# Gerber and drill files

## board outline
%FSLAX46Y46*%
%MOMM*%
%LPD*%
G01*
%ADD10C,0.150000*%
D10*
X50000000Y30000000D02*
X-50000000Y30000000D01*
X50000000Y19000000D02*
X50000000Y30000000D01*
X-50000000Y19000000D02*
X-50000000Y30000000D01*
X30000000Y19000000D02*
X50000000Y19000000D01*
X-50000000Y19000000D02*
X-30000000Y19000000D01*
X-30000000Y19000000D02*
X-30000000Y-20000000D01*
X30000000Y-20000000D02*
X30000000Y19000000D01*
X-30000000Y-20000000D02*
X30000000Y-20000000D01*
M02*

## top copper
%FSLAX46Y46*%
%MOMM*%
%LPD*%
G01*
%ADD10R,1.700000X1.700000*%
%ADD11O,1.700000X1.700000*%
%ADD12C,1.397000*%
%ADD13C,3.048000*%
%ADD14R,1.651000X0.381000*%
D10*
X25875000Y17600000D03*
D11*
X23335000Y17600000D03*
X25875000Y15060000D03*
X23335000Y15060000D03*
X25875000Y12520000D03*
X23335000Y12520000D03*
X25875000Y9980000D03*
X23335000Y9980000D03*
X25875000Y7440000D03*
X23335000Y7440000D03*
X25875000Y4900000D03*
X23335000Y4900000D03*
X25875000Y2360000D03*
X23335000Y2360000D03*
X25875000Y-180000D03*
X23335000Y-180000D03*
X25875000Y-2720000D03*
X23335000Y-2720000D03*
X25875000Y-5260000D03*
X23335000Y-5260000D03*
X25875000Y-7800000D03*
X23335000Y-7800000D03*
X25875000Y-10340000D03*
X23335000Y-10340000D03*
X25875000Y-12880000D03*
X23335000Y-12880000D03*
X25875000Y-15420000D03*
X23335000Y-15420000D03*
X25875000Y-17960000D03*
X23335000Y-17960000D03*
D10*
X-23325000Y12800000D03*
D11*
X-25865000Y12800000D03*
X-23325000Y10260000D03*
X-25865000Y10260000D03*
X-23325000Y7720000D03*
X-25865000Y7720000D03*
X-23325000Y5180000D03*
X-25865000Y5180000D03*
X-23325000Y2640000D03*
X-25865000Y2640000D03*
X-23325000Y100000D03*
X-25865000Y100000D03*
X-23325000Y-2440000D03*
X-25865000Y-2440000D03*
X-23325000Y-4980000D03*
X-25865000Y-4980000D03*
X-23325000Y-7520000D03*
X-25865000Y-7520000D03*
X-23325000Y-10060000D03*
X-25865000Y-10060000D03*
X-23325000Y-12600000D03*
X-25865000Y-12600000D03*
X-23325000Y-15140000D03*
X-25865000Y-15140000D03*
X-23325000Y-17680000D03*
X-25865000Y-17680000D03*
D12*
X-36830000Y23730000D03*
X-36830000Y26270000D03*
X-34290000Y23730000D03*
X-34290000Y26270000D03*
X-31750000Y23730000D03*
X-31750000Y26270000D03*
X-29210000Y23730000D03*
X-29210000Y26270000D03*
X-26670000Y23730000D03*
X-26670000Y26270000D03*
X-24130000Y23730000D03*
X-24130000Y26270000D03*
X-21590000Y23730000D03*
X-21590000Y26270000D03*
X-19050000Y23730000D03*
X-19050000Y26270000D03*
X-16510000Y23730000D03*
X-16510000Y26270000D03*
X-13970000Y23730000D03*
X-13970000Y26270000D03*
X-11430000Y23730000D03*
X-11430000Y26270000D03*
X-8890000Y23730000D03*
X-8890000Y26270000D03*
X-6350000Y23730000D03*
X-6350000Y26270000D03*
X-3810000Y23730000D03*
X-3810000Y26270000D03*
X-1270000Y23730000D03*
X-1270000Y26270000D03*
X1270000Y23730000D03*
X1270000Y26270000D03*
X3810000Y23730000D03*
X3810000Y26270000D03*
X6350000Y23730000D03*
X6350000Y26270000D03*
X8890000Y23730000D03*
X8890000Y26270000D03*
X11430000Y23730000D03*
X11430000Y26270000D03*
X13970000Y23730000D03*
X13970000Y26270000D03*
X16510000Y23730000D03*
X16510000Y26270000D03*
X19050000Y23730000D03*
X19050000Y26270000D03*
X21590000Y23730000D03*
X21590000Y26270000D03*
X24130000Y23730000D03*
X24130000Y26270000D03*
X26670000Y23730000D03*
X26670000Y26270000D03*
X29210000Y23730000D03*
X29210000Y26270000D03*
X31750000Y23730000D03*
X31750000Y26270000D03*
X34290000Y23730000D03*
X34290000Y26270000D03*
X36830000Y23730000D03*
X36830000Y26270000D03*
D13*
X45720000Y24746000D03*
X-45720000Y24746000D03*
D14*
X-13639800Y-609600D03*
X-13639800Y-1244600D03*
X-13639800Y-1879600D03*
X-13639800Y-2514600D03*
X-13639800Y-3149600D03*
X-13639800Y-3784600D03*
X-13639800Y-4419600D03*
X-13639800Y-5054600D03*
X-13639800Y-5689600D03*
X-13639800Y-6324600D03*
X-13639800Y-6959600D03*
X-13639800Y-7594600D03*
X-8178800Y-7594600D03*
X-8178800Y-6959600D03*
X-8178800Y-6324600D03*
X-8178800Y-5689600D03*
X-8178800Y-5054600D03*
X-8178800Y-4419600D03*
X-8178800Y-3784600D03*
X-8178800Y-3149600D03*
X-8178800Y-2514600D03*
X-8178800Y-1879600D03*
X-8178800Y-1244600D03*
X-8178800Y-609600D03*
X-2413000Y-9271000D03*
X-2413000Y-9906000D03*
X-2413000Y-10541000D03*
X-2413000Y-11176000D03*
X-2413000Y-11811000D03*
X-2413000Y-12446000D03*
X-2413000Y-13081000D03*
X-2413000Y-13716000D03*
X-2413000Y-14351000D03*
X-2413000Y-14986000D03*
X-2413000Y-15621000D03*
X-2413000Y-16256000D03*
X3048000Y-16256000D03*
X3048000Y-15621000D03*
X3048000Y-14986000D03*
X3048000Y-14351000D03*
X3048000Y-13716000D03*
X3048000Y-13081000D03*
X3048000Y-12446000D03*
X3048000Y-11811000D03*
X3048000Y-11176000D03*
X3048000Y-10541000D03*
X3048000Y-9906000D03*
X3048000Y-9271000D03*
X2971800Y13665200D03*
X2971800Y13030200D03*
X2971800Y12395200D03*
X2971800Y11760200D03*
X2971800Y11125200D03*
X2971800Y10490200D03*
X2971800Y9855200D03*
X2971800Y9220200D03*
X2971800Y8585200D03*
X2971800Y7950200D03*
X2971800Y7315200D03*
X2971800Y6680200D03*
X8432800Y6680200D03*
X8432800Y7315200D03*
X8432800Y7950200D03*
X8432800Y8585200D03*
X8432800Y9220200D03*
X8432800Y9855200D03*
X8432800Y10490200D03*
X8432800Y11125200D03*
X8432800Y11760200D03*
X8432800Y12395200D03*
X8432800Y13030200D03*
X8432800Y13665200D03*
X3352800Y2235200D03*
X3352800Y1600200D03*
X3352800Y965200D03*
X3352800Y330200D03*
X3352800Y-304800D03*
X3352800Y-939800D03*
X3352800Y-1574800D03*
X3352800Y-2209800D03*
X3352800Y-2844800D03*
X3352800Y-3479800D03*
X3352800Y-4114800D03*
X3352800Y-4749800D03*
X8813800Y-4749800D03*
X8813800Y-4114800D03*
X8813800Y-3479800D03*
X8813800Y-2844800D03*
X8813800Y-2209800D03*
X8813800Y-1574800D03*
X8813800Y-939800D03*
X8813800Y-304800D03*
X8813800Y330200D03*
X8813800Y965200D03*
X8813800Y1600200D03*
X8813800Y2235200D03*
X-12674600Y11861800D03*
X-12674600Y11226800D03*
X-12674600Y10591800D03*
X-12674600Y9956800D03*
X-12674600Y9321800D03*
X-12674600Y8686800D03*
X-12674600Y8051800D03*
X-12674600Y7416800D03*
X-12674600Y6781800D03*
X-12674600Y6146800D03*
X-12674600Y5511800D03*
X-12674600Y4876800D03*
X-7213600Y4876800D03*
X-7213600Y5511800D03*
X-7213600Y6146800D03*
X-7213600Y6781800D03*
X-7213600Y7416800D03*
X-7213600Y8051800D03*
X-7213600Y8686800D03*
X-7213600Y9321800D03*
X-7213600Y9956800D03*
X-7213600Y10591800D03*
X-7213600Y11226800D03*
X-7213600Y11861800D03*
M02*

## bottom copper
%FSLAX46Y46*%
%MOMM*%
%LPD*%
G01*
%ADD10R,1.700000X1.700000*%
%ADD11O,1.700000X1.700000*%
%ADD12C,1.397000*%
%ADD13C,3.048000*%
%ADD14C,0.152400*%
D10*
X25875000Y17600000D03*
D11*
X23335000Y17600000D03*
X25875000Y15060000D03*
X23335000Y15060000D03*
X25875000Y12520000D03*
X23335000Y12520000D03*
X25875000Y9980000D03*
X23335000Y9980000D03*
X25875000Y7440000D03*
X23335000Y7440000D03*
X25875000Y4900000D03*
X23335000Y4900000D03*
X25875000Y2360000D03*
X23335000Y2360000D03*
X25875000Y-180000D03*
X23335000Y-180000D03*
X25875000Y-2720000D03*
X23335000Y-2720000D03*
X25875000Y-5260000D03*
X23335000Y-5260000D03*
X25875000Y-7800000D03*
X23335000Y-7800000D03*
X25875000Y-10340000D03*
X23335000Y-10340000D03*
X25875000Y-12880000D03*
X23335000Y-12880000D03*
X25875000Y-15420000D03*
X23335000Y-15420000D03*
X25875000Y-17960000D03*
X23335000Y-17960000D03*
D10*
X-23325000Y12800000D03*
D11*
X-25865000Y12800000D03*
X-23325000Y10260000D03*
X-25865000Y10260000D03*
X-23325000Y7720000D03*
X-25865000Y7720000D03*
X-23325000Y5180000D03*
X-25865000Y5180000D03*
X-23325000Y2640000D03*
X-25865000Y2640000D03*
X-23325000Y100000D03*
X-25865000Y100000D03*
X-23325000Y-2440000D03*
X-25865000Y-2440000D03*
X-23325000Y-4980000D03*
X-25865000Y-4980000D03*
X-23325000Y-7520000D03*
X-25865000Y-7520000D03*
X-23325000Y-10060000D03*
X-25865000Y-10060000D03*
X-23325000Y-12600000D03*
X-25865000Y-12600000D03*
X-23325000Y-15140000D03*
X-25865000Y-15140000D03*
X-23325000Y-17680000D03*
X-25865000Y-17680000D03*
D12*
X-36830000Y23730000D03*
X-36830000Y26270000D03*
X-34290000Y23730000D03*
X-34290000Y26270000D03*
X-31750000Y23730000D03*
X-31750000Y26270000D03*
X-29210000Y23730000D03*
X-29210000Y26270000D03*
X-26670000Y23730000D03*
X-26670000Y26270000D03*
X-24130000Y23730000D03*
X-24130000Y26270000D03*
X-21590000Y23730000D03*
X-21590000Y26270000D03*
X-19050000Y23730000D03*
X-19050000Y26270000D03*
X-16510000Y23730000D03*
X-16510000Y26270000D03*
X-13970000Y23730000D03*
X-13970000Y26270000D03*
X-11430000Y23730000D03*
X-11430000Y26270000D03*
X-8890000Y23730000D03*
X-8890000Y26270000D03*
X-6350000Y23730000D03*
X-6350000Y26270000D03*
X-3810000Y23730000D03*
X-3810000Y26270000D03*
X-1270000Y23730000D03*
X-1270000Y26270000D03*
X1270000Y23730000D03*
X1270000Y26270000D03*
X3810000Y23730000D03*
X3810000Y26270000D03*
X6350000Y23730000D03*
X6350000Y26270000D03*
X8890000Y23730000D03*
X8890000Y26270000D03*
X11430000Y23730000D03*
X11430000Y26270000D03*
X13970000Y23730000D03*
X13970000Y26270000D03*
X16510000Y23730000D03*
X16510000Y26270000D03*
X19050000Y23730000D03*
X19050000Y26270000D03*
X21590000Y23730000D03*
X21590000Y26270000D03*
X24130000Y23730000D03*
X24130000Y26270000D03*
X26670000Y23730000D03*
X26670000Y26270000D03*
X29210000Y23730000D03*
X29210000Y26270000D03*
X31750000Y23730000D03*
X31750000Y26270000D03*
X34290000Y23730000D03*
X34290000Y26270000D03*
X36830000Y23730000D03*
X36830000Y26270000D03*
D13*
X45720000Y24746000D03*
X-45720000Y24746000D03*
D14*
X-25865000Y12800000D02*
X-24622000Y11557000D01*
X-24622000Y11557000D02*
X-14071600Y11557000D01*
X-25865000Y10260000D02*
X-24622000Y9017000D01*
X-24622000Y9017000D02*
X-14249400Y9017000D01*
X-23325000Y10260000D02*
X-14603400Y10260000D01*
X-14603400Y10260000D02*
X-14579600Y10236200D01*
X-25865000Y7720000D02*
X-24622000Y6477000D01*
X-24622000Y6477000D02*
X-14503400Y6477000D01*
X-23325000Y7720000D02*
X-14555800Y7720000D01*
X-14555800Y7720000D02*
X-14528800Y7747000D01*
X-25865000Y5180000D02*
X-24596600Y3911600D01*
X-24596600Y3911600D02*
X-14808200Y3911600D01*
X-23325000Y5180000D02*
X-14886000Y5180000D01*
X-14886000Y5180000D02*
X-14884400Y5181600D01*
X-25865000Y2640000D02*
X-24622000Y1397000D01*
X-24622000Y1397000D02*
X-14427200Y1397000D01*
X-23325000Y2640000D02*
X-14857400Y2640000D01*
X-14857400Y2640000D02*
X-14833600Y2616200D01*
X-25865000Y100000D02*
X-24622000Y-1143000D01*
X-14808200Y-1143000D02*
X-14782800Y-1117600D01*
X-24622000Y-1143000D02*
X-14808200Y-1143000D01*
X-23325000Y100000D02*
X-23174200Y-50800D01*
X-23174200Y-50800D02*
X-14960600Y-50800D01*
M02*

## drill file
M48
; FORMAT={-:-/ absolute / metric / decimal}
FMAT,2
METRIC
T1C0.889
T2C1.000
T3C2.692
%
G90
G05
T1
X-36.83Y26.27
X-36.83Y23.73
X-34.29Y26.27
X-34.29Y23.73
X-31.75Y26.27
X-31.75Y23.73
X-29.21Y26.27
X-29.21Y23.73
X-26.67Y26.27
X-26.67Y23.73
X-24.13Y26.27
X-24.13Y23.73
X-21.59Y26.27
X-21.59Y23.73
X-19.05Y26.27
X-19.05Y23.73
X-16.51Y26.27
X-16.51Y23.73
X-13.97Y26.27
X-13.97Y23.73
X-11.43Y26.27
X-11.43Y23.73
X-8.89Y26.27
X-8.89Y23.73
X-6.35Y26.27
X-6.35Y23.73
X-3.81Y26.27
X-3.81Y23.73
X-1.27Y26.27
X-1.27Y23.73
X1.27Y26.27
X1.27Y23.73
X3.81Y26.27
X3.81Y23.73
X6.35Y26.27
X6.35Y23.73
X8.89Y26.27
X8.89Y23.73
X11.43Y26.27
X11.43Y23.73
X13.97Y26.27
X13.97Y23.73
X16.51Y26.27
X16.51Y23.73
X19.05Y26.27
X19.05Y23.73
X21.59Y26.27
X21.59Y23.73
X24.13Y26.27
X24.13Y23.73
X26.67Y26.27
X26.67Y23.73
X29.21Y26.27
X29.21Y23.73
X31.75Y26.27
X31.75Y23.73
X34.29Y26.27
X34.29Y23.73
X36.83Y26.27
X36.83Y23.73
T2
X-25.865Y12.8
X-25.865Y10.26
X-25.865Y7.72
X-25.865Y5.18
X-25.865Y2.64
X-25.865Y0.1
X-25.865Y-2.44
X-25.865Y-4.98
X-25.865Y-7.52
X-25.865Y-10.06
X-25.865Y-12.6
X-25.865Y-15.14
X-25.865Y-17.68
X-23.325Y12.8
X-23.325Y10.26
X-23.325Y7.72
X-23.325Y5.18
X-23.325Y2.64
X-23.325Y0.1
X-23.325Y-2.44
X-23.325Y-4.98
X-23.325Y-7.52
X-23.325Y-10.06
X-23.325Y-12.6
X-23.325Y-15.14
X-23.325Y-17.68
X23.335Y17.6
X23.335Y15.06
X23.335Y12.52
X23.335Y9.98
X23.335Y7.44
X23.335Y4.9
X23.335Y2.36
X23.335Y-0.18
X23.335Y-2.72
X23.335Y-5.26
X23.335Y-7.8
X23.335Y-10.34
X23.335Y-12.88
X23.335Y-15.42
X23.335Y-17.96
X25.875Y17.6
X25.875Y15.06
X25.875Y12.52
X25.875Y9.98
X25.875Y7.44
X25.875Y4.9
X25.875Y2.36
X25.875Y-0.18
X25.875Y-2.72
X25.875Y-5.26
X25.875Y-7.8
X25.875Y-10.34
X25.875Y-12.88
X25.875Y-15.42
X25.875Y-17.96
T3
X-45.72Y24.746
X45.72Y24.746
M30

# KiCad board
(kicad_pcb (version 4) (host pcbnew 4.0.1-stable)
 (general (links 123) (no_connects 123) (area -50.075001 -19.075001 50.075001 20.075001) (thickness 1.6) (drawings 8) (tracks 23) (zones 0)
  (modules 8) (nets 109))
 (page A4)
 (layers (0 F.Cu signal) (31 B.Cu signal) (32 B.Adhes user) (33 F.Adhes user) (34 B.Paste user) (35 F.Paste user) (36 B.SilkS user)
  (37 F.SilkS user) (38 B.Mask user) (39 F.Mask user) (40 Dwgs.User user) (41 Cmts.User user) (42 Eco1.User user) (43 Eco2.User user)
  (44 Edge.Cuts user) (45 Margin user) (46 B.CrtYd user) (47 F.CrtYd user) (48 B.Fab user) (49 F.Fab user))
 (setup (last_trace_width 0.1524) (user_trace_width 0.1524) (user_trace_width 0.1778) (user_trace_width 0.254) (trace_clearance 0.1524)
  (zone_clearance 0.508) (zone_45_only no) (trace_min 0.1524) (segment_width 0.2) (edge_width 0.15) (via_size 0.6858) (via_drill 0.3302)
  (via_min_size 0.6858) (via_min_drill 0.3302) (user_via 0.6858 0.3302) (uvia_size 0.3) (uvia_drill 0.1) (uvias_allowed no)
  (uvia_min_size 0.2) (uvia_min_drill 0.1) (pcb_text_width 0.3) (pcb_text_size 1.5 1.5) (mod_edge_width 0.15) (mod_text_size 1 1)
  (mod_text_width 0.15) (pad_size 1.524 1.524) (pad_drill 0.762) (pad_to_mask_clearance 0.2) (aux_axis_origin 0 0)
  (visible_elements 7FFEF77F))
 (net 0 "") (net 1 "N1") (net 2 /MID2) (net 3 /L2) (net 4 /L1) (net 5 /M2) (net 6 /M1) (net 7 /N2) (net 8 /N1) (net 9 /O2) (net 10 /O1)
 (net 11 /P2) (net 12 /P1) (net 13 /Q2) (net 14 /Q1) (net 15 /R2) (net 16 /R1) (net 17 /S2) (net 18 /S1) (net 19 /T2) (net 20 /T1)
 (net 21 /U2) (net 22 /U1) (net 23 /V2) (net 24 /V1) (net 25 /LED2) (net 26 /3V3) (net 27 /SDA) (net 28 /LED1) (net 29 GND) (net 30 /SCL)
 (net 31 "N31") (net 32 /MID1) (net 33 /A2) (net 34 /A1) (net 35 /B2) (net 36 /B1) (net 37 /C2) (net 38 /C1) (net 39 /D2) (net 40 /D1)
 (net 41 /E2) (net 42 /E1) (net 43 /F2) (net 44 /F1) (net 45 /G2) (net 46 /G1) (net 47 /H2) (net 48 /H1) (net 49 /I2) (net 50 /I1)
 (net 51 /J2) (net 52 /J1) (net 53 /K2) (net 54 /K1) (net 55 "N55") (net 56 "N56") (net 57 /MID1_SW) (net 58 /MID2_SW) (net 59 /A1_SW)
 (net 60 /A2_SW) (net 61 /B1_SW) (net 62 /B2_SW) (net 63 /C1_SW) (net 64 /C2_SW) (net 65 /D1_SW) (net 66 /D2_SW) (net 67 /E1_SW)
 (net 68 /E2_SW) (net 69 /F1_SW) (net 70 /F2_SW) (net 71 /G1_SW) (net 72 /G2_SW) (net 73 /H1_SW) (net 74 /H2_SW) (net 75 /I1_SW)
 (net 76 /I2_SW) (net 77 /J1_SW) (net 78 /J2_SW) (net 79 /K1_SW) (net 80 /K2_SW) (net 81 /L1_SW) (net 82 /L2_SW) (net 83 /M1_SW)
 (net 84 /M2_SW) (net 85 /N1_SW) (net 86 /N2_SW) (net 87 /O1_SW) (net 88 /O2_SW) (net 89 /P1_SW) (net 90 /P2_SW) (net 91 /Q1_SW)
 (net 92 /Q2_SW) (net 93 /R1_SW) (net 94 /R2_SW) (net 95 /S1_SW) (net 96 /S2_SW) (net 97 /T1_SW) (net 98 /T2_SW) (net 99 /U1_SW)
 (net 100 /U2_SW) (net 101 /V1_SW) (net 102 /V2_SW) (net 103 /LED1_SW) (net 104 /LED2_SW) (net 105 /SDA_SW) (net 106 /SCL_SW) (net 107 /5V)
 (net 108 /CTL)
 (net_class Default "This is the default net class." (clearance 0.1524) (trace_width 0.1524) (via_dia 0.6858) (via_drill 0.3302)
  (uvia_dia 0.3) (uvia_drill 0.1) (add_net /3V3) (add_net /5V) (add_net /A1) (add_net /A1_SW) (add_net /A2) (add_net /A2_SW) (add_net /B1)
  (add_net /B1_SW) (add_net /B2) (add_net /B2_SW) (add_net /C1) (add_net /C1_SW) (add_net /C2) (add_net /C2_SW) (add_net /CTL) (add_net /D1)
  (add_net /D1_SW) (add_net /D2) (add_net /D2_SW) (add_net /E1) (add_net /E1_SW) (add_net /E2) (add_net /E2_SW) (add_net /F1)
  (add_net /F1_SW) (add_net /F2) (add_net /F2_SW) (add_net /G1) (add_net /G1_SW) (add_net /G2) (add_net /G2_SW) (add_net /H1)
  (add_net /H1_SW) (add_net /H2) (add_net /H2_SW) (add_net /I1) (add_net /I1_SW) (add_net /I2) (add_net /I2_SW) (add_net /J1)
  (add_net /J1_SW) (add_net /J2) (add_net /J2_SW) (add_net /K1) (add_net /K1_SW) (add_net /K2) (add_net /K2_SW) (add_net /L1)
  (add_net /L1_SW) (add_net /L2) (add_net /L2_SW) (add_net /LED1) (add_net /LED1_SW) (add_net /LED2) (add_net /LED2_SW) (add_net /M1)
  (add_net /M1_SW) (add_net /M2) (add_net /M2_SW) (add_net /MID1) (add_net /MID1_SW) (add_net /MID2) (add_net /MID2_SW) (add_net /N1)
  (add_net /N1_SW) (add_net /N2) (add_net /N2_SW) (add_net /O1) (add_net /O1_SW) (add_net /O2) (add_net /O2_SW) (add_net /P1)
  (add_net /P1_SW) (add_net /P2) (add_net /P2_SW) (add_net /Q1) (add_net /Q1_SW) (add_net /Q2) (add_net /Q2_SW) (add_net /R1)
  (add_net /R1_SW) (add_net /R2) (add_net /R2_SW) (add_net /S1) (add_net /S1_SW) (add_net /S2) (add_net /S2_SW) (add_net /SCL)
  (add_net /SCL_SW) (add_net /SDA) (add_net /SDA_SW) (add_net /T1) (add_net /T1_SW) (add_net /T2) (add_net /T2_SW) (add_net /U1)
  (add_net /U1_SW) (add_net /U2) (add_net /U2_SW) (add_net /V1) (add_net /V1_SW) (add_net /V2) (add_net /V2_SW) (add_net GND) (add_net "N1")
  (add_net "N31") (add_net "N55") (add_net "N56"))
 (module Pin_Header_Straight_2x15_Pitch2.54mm (layer B.Cu) (at 24.605 0.18 180)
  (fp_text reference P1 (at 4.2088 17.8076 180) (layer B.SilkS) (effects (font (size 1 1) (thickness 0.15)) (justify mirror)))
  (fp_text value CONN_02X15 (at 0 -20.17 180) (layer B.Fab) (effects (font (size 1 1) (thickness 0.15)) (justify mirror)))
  (pad 1 thru_hole rect (at -1.27 17.78 180) (size 1.7 1.7) (drill 1) (layers *.Cu *.Mask) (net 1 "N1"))
  (pad 2 thru_hole oval (at 1.27 17.78 180) (size 1.7 1.7) (drill 1) (layers *.Cu *.Mask) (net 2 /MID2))
  (pad 3 thru_hole oval (at -1.27 15.24 180) (size 1.7 1.7) (drill 1) (layers *.Cu *.Mask) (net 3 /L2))
  (pad 4 thru_hole oval (at 1.27 15.24 180) (size 1.7 1.7) (drill 1) (layers *.Cu *.Mask) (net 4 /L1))
  (pad 5 thru_hole oval (at -1.27 12.7 180) (size 1.7 1.7) (drill 1) (layers *.Cu *.Mask) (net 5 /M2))
  (pad 6 thru_hole oval (at 1.27 12.7 180) (size 1.7 1.7) (drill 1) (layers *.Cu *.Mask) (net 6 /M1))
  (pad 7 thru_hole oval (at -1.27 10.16 180) (size 1.7 1.7) (drill 1) (layers *.Cu *.Mask) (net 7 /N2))
  (pad 8 thru_hole oval (at 1.27 10.16 180) (size 1.7 1.7) (drill 1) (layers *.Cu *.Mask) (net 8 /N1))
  (pad 9 thru_hole oval (at -1.27 7.62 180) (size 1.7 1.7) (drill 1) (layers *.Cu *.Mask) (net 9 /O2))
  (pad 10 thru_hole oval (at 1.27 7.62 180) (size 1.7 1.7) (drill 1) (layers *.Cu *.Mask) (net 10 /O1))
  (pad 11 thru_hole oval (at -1.27 5.08 180) (size 1.7 1.7) (drill 1) (layers *.Cu *.Mask) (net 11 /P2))
  (pad 12 thru_hole oval (at 1.27 5.08 180) (size 1.7 1.7) (drill 1) (layers *.Cu *.Mask) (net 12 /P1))
  (pad 13 thru_hole oval (at -1.27 2.54 180) (size 1.7 1.7) (drill 1) (layers *.Cu *.Mask) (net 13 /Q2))
  (pad 14 thru_hole oval (at 1.27 2.54 180) (size 1.7 1.7) (drill 1) (layers *.Cu *.Mask) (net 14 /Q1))
  (pad 15 thru_hole oval (at -1.27 0 180) (size 1.7 1.7) (drill 1) (layers *.Cu *.Mask) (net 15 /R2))
  (pad 16 thru_hole oval (at 1.27 0 180) (size 1.7 1.7) (drill 1) (layers *.Cu *.Mask) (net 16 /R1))
  (pad 17 thru_hole oval (at -1.27 -2.54 180) (size 1.7 1.7) (drill 1) (layers *.Cu *.Mask) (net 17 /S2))
  (pad 18 thru_hole oval (at 1.27 -2.54 180) (size 1.7 1.7) (drill 1) (layers *.Cu *.Mask) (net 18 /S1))
  (pad 19 thru_hole oval (at -1.27 -5.08 180) (size 1.7 1.7) (drill 1) (layers *.Cu *.Mask) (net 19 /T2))
  (pad 20 thru_hole oval (at 1.27 -5.08 180) (size 1.7 1.7) (drill 1) (layers *.Cu *.Mask) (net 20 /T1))
  (pad 21 thru_hole oval (at -1.27 -7.62 180) (size 1.7 1.7) (drill 1) (layers *.Cu *.Mask) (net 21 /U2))
  (pad 22 thru_hole oval (at 1.27 -7.62 180) (size 1.7 1.7) (drill 1) (layers *.Cu *.Mask) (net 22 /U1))
  (pad 23 thru_hole oval (at -1.27 -10.16 180) (size 1.7 1.7) (drill 1) (layers *.Cu *.Mask) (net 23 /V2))
  (pad 24 thru_hole oval (at 1.27 -10.16 180) (size 1.7 1.7) (drill 1) (layers *.Cu *.Mask) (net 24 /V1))
  (pad 25 thru_hole oval (at -1.27 -12.7 180) (size 1.7 1.7) (drill 1) (layers *.Cu *.Mask) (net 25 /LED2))
  (pad 26 thru_hole oval (at 1.27 -12.7 180) (size 1.7 1.7) (drill 1) (layers *.Cu *.Mask) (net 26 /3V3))
  (pad 27 thru_hole oval (at -1.27 -15.24 180) (size 1.7 1.7) (drill 1) (layers *.Cu *.Mask) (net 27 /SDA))
  (pad 28 thru_hole oval (at 1.27 -15.24 180) (size 1.7 1.7) (drill 1) (layers *.Cu *.Mask) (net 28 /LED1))
  (pad 29 thru_hole oval (at -1.27 -17.78 180) (size 1.7 1.7) (drill 1) (layers *.Cu *.Mask) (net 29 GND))
  (pad 30 thru_hole oval (at 1.27 -17.78 180) (size 1.7 1.7) (drill 1) (layers *.Cu *.Mask) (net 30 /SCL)))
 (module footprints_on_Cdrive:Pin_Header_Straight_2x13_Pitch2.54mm (layer B.Cu) (at -24.595 2.44 180)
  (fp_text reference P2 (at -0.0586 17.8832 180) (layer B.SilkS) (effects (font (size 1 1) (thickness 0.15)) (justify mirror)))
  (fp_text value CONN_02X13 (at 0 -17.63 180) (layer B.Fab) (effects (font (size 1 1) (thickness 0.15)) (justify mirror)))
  (pad 1 thru_hole rect (at -1.27 15.24 180) (size 1.7 1.7) (drill 1) (layers *.Cu *.Mask) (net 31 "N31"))
  (pad 2 thru_hole oval (at 1.27 15.24 180) (size 1.7 1.7) (drill 1) (layers *.Cu *.Mask) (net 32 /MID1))
  (pad 3 thru_hole oval (at -1.27 12.7 180) (size 1.7 1.7) (drill 1) (layers *.Cu *.Mask) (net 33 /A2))
  (pad 4 thru_hole oval (at 1.27 12.7 180) (size 1.7 1.7) (drill 1) (layers *.Cu *.Mask) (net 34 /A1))
  (pad 5 thru_hole oval (at -1.27 10.16 180) (size 1.7 1.7) (drill 1) (layers *.Cu *.Mask) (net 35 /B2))
  (pad 6 thru_hole oval (at 1.27 10.16 180) (size 1.7 1.7) (drill 1) (layers *.Cu *.Mask) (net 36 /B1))
  (pad 7 thru_hole oval (at -1.27 7.62 180) (size 1.7 1.7) (drill 1) (layers *.Cu *.Mask) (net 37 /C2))
  (pad 8 thru_hole oval (at 1.27 7.62 180) (size 1.7 1.7) (drill 1) (layers *.Cu *.Mask) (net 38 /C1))
  (pad 9 thru_hole oval (at -1.27 5.08 180) (size 1.7 1.7) (drill 1) (layers *.Cu *.Mask) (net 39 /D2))
  (pad 10 thru_hole oval (at 1.27 5.08 180) (size 1.7 1.7) (drill 1) (layers *.Cu *.Mask) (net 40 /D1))
  (pad 11 thru_hole oval (at -1.27 2.54 180) (size 1.7 1.7) (drill 1) (layers *.Cu *.Mask) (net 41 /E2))
  (pad 12 thru_hole oval (at 1.27 2.54 180) (size 1.7 1.7) (drill 1) (layers *.Cu *.Mask) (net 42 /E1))
  (pad 13 thru_hole oval (at -1.27 0 180) (size 1.7 1.7) (drill 1) (layers *.Cu *.Mask) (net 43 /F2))
  (pad 14 thru_hole oval (at 1.27 0 180) (size 1.7 1.7) (drill 1) (layers *.Cu *.Mask) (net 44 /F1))
  (pad 15 thru_hole oval (at -1.27 -2.54 180) (size 1.7 1.7) (drill 1) (layers *.Cu *.Mask) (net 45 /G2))
  (pad 16 thru_hole oval (at 1.27 -2.54 180) (size 1.7 1.7) (drill 1) (layers *.Cu *.Mask) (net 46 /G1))
  (pad 17 thru_hole oval (at -1.27 -5.08 180) (size 1.7 1.7) (drill 1) (layers *.Cu *.Mask) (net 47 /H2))
  (pad 18 thru_hole oval (at 1.27 -5.08 180) (size 1.7 1.7) (drill 1) (layers *.Cu *.Mask) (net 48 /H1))
  (pad 19 thru_hole oval (at -1.27 -7.62 180) (size 1.7 1.7) (drill 1) (layers *.Cu *.Mask) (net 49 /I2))
  (pad 20 thru_hole oval (at 1.27 -7.62 180) (size 1.7 1.7) (drill 1) (layers *.Cu *.Mask) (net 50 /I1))
  (pad 21 thru_hole oval (at -1.27 -10.16 180) (size 1.7 1.7) (drill 1) (layers *.Cu *.Mask) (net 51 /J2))
  (pad 22 thru_hole oval (at 1.27 -10.16 180) (size 1.7 1.7) (drill 1) (layers *.Cu *.Mask) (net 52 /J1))
  (pad 23 thru_hole oval (at -1.27 -12.7 180) (size 1.7 1.7) (drill 1) (layers *.Cu *.Mask) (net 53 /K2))
  (pad 24 thru_hole oval (at 1.27 -12.7 180) (size 1.7 1.7) (drill 1) (layers *.Cu *.Mask) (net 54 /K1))
  (pad 25 thru_hole oval (at -1.27 -15.24 180) (size 1.7 1.7) (drill 1) (layers *.Cu *.Mask) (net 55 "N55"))
  (pad 26 thru_hole oval (at 1.27 -15.24 180) (size 1.7 1.7) (drill 1) (layers *.Cu *.Mask) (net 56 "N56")))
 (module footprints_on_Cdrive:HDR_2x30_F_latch (layer F.Cu) (at 0 -25)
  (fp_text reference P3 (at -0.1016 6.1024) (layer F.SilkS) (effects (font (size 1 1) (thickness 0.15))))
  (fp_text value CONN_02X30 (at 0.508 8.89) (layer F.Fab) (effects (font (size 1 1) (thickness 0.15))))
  (pad 1 thru_hole circle (at -36.83 1.27) (size 1.397 1.397) (drill 0.889) (layers *.Cu *.Mask F.SilkS) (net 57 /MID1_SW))
  (pad 2 thru_hole circle (at -36.83 -1.27) (size 1.397 1.397) (drill 0.889) (layers *.Cu *.Mask F.SilkS) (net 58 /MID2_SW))
  (pad 3 thru_hole circle (at -34.29 1.27) (size 1.397 1.397) (drill 0.889) (layers *.Cu *.Mask F.SilkS) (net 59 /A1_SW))
  (pad 4 thru_hole circle (at -34.29 -1.27) (size 1.397 1.397) (drill 0.889) (layers *.Cu *.Mask F.SilkS) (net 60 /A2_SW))
  (pad 5 thru_hole circle (at -31.75 1.27) (size 1.397 1.397) (drill 0.889) (layers *.Cu *.Mask F.SilkS) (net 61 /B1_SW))
  (pad 6 thru_hole circle (at -31.75 -1.27) (size 1.397 1.397) (drill 0.889) (layers *.Cu *.Mask F.SilkS) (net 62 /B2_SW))
  (pad 7 thru_hole circle (at -29.21 1.27) (size 1.397 1.397) (drill 0.889) (layers *.Cu *.Mask F.SilkS) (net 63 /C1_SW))
  (pad 8 thru_hole circle (at -29.21 -1.27) (size 1.397 1.397) (drill 0.889) (layers *.Cu *.Mask F.SilkS) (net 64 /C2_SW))
  (pad 9 thru_hole circle (at -26.67 1.27) (size 1.397 1.397) (drill 0.889) (layers *.Cu *.Mask F.SilkS) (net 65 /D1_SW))
  (pad 10 thru_hole circle (at -26.67 -1.27) (size 1.397 1.397) (drill 0.889) (layers *.Cu *.Mask F.SilkS) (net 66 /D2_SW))
  (pad 11 thru_hole circle (at -24.13 1.27) (size 1.397 1.397) (drill 0.889) (layers *.Cu *.Mask F.SilkS) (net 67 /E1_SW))
  (pad 12 thru_hole circle (at -24.13 -1.27) (size 1.397 1.397) (drill 0.889) (layers *.Cu *.Mask F.SilkS) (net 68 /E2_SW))
  (pad 13 thru_hole circle (at -21.59 1.27) (size 1.397 1.397) (drill 0.889) (layers *.Cu *.Mask F.SilkS) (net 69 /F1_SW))
  (pad 14 thru_hole circle (at -21.59 -1.27) (size 1.397 1.397) (drill 0.889) (layers *.Cu *.Mask F.SilkS) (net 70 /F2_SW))
  (pad 15 thru_hole circle (at -19.05 1.27) (size 1.397 1.397) (drill 0.889) (layers *.Cu *.Mask F.SilkS) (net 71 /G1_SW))
  (pad 16 thru_hole circle (at -19.05 -1.27) (size 1.397 1.397) (drill 0.889) (layers *.Cu *.Mask F.SilkS) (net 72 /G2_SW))
  (pad 17 thru_hole circle (at -16.51 1.27) (size 1.397 1.397) (drill 0.889) (layers *.Cu *.Mask F.SilkS) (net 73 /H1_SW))
  (pad 18 thru_hole circle (at -16.51 -1.27) (size 1.397 1.397) (drill 0.889) (layers *.Cu *.Mask F.SilkS) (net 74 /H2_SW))
  (pad 19 thru_hole circle (at -13.97 1.27) (size 1.397 1.397) (drill 0.889) (layers *.Cu *.Mask F.SilkS) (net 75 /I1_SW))
  (pad 20 thru_hole circle (at -13.97 -1.27) (size 1.397 1.397) (drill 0.889) (layers *.Cu *.Mask F.SilkS) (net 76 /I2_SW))
  (pad 21 thru_hole circle (at -11.43 1.27) (size 1.397 1.397) (drill 0.889) (layers *.Cu *.Mask F.SilkS) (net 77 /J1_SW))
  (pad 22 thru_hole circle (at -11.43 -1.27) (size 1.397 1.397) (drill 0.889) (layers *.Cu *.Mask F.SilkS) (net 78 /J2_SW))
  (pad 23 thru_hole circle (at -8.89 1.27) (size 1.397 1.397) (drill 0.889) (layers *.Cu *.Mask F.SilkS) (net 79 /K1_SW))
  (pad 24 thru_hole circle (at -8.89 -1.27) (size 1.397 1.397) (drill 0.889) (layers *.Cu *.Mask F.SilkS) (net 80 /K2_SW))
  (pad 25 thru_hole circle (at -6.35 1.27) (size 1.397 1.397) (drill 0.889) (layers *.Cu *.Mask F.SilkS) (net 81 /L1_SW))
  (pad 26 thru_hole circle (at -6.35 -1.27) (size 1.397 1.397) (drill 0.889) (layers *.Cu *.Mask F.SilkS) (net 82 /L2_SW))
  (pad 27 thru_hole circle (at -3.81 1.27) (size 1.397 1.397) (drill 0.889) (layers *.Cu *.Mask F.SilkS) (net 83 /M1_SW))
  (pad 28 thru_hole circle (at -3.81 -1.27) (size 1.397 1.397) (drill 0.889) (layers *.Cu *.Mask F.SilkS) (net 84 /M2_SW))
  (pad 29 thru_hole circle (at -1.27 1.27) (size 1.397 1.397) (drill 0.889) (layers *.Cu *.Mask F.SilkS) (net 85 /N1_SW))
  (pad 30 thru_hole circle (at -1.27 -1.27) (size 1.397 1.397) (drill 0.889) (layers *.Cu *.Mask F.SilkS) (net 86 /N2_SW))
  (pad 31 thru_hole circle (at 1.27 1.27) (size 1.397 1.397) (drill 0.889) (layers *.Cu *.Mask F.SilkS) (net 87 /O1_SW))
  (pad 32 thru_hole circle (at 1.27 -1.27) (size 1.397 1.397) (drill 0.889) (layers *.Cu *.Mask F.SilkS) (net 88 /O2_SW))
  (pad 33 thru_hole circle (at 3.81 1.27) (size 1.397 1.397) (drill 0.889) (layers *.Cu *.Mask F.SilkS) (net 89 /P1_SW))
  (pad 34 thru_hole circle (at 3.81 -1.27) (size 1.397 1.397) (drill 0.889) (layers *.Cu *.Mask F.SilkS) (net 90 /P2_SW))
  (pad 35 thru_hole circle (at 6.35 1.27) (size 1.397 1.397) (drill 0.889) (layers *.Cu *.Mask F.SilkS) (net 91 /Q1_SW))
  (pad 36 thru_hole circle (at 6.35 -1.27) (size 1.397 1.397) (drill 0.889) (layers *.Cu *.Mask F.SilkS) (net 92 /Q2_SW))
  (pad 37 thru_hole circle (at 8.89 1.27) (size 1.397 1.397) (drill 0.889) (layers *.Cu *.Mask F.SilkS) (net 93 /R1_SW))
  (pad 38 thru_hole circle (at 8.89 -1.27) (size 1.397 1.397) (drill 0.889) (layers *.Cu *.Mask F.SilkS) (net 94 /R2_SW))
  (pad 39 thru_hole circle (at 11.43 1.27) (size 1.397 1.397) (drill 0.889) (layers *.Cu *.Mask F.SilkS) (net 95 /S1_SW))
  (pad 40 thru_hole circle (at 11.43 -1.27) (size 1.397 1.397) (drill 0.889) (layers *.Cu *.Mask F.SilkS) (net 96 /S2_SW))
  (pad 41 thru_hole circle (at 13.97 1.27) (size 1.397 1.397) (drill 0.889) (layers *.Cu *.Mask F.SilkS) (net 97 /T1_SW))
  (pad 42 thru_hole circle (at 13.97 -1.27) (size 1.397 1.397) (drill 0.889) (layers *.Cu *.Mask F.SilkS) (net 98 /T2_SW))
  (pad 43 thru_hole circle (at 16.51 1.27) (size 1.397 1.397) (drill 0.889) (layers *.Cu *.Mask F.SilkS) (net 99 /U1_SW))
  (pad 44 thru_hole circle (at 16.51 -1.27) (size 1.397 1.397) (drill 0.889) (layers *.Cu *.Mask F.SilkS) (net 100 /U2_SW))
  (pad 45 thru_hole circle (at 19.05 1.27) (size 1.397 1.397) (drill 0.889) (layers *.Cu *.Mask F.SilkS) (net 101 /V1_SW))
  (pad 46 thru_hole circle (at 19.05 -1.27) (size 1.397 1.397) (drill 0.889) (layers *.Cu *.Mask F.SilkS) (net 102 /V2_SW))
  (pad 47 thru_hole circle (at 21.59 1.27) (size 1.397 1.397) (drill 0.889) (layers *.Cu *.Mask F.SilkS) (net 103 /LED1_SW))
  (pad 48 thru_hole circle (at 21.59 -1.27) (size 1.397 1.397) (drill 0.889) (layers *.Cu *.Mask F.SilkS) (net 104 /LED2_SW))
  (pad 49 thru_hole circle (at 24.13 1.27) (size 1.397 1.397) (drill 0.889) (layers *.Cu *.Mask F.SilkS) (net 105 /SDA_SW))
  (pad 50 thru_hole circle (at 24.13 -1.27) (size 1.397 1.397) (drill 0.889) (layers *.Cu *.Mask F.SilkS) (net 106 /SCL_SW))
  (pad 51 thru_hole circle (at 26.67 1.27) (size 1.397 1.397) (drill 0.889) (layers *.Cu *.Mask F.SilkS) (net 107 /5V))
  (pad 52 thru_hole circle (at 26.67 -1.27) (size 1.397 1.397) (drill 0.889) (layers *.Cu *.Mask F.SilkS) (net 107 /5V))
  (pad 53 thru_hole circle (at 29.21 1.27) (size 1.397 1.397) (drill 0.889) (layers *.Cu *.Mask F.SilkS) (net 107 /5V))
  (pad 54 thru_hole circle (at 29.21 -1.27) (size 1.397 1.397) (drill 0.889) (layers *.Cu *.Mask F.SilkS) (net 26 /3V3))
  (pad 55 thru_hole circle (at 31.75 1.27) (size 1.397 1.397) (drill 0.889) (layers *.Cu *.Mask F.SilkS) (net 26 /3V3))
  (pad 56 thru_hole circle (at 31.75 -1.27) (size 1.397 1.397) (drill 0.889) (layers *.Cu *.Mask F.SilkS) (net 26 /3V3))
  (pad 57 thru_hole circle (at 34.29 1.27) (size 1.397 1.397) (drill 0.889) (layers *.Cu *.Mask F.SilkS) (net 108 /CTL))
  (pad 58 thru_hole circle (at 34.29 -1.27) (size 1.397 1.397) (drill 0.889) (layers *.Cu *.Mask F.SilkS) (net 29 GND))
  (pad 59 thru_hole circle (at 36.83 1.27) (size 1.397 1.397) (drill 0.889) (layers *.Cu *.Mask F.SilkS) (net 29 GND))
  (pad 60 thru_hole circle (at 36.83 -1.27) (size 1.397 1.397) (drill 0.889) (layers *.Cu *.Mask F.SilkS) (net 29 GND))
  (pad 0 thru_hole circle (at 45.72 0.254) (size 3.048 3.048) (drill 2.6924) (layers *.Cu *.Mask F.SilkS))
  (pad 0 thru_hole circle (at -45.72 0.254) (size 3.048 3.048) (drill 2.6924) (layers *.Cu *.Mask F.SilkS)))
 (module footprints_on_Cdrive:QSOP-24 (layer F.Cu) (at -13.6398 0.6096 270)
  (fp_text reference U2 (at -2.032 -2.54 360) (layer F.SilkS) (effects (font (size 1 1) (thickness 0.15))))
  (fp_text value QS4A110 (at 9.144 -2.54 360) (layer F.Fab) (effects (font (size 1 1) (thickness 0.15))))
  (pad 1 smd rect (at 0 0 270) (size 0.381 1.651) (layers F.Cu F.Paste F.Mask) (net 108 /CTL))
  (pad 2 smd rect (at 0.635 0 270) (size 0.381 1.651) (layers F.Cu F.Paste F.Mask) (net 67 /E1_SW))
  (pad 3 smd rect (at 1.27 0 270) (size 0.381 1.651) (layers F.Cu F.Paste F.Mask) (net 42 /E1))
  (pad 4 smd rect (at 1.905 0 270) (size 0.381 1.651) (layers F.Cu F.Paste F.Mask) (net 41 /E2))
  (pad 5 smd rect (at 2.54 0 270) (size 0.381 1.651) (layers F.Cu F.Paste F.Mask) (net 72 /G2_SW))
  (pad 6 smd rect (at 3.175 0 270) (size 0.381 1.651) (layers F.Cu F.Paste F.Mask) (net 69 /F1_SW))
  (pad 7 smd rect (at 3.81 0 270) (size 0.381 1.651) (layers F.Cu F.Paste F.Mask) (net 44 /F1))
  (pad 8 smd rect (at 4.445 0 270) (size 0.381 1.651) (layers F.Cu F.Paste F.Mask) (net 43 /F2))
  (pad 9 smd rect (at 5.08 0 270) (size 0.381 1.651) (layers F.Cu F.Paste F.Mask) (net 70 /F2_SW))
  (pad 10 smd rect (at 5.715 0 270) (size 0.381 1.651) (layers F.Cu F.Paste F.Mask) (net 71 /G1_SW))
  (pad 11 smd rect (at 6.35 0 270) (size 0.381 1.651) (layers F.Cu F.Paste F.Mask) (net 46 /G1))
  (pad 12 smd rect (at 6.985 0 270) (size 0.381 1.651) (layers F.Cu F.Paste F.Mask) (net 29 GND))
  (pad 13 smd rect (at 6.985 -5.461 270) (size 0.381 1.651) (layers F.Cu F.Paste F.Mask) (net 108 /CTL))
  (pad 14 smd rect (at 6.35 -5.461 270) (size 0.381 1.651) (layers F.Cu F.Paste F.Mask) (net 45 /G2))
  (pad 15 smd rect (at 5.715 -5.461 270) (size 0.381 1.651) (layers F.Cu F.Paste F.Mask))
  (pad 16 smd rect (at 5.08 -5.461 270) (size 0.381 1.651) (layers F.Cu F.Paste F.Mask) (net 73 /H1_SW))
  (pad 17 smd rect (at 4.445 -5.461 270) (size 0.381 1.651) (layers F.Cu F.Paste F.Mask) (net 48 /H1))
  (pad 18 smd rect (at 3.81 -5.461 270) (size 0.381 1.651) (layers F.Cu F.Paste F.Mask) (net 47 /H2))
  (pad 19 smd rect (at 3.175 -5.461 270) (size 0.381 1.651) (layers F.Cu F.Paste F.Mask) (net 74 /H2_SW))
  (pad 20 smd rect (at 2.54 -5.461 270) (size 0.381 1.651) (layers F.Cu F.Paste F.Mask) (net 75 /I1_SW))
  (pad 21 smd rect (at 1.905 -5.461 270) (size 0.381 1.651) (layers F.Cu F.Paste F.Mask) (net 50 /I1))
  (pad 22 smd rect (at 1.27 -5.461 270) (size 0.381 1.651) (layers F.Cu F.Paste F.Mask) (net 49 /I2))
  (pad 23 smd rect (at 0.635 -5.461 270) (size 0.381 1.651) (layers F.Cu F.Paste F.Mask) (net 76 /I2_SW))
  (pad 24 smd rect (at 0 -5.461 270) (size 0.381 1.651) (layers F.Cu F.Paste F.Mask) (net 107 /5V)))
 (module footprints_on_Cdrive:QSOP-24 (layer F.Cu) (at -2.413 9.271 270)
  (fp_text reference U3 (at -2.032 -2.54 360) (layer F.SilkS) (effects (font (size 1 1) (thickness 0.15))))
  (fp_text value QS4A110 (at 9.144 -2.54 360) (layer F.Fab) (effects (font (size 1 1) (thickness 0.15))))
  (pad 1 smd rect (at 0 0 270) (size 0.381 1.651) (layers F.Cu F.Paste F.Mask) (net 108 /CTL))
  (pad 2 smd rect (at 0.635 0 270) (size 0.381 1.651) (layers F.Cu F.Paste F.Mask) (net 77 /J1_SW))
  (pad 3 smd rect (at 1.27 0 270) (size 0.381 1.651) (layers F.Cu F.Paste F.Mask) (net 52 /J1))
  (pad 4 smd rect (at 1.905 0 270) (size 0.381 1.651) (layers F.Cu F.Paste F.Mask) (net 51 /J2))
  (pad 5 smd rect (at 2.54 0 270) (size 0.381 1.651) (layers F.Cu F.Paste F.Mask) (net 78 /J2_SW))
  (pad 6 smd rect (at 3.175 0 270) (size 0.381 1.651) (layers F.Cu F.Paste F.Mask) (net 79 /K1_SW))
  (pad 7 smd rect (at 3.81 0 270) (size 0.381 1.651) (layers F.Cu F.Paste F.Mask) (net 54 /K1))
  (pad 8 smd rect (at 4.445 0 270) (size 0.381 1.651) (layers F.Cu F.Paste F.Mask) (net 53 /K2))
  (pad 9 smd rect (at 5.08 0 270) (size 0.381 1.651) (layers F.Cu F.Paste F.Mask) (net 80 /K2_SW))
  (pad 10 smd rect (at 5.715 0 270) (size 0.381 1.651) (layers F.Cu F.Paste F.Mask) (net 81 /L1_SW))
  (pad 11 smd rect (at 6.35 0 270) (size 0.381 1.651) (layers F.Cu F.Paste F.Mask) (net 4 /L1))
  (pad 12 smd rect (at 6.985 0 270) (size 0.381 1.651) (layers F.Cu F.Paste F.Mask) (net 29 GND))
  (pad 13 smd rect (at 6.985 -5.461 270) (size 0.381 1.651) (layers F.Cu F.Paste F.Mask) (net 108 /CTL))
  (pad 14 smd rect (at 6.35 -5.461 270) (size 0.381 1.651) (layers F.Cu F.Paste F.Mask) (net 3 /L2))
  (pad 15 smd rect (at 5.715 -5.461 270) (size 0.381 1.651) (layers F.Cu F.Paste F.Mask))
  (pad 16 smd rect (at 5.08 -5.461 270) (size 0.381 1.651) (layers F.Cu F.Paste F.Mask) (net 83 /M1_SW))
  (pad 17 smd rect (at 4.445 -5.461 270) (size 0.381 1.651) (layers F.Cu F.Paste F.Mask) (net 6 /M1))
  (pad 18 smd rect (at 3.81 -5.461 270) (size 0.381 1.651) (layers F.Cu F.Paste F.Mask) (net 5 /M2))
  (pad 19 smd rect (at 3.175 -5.461 270) (size 0.381 1.651) (layers F.Cu F.Paste F.Mask) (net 84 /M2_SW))
  (pad 20 smd rect (at 2.54 -5.461 270) (size 0.381 1.651) (layers F.Cu F.Paste F.Mask) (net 85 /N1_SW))
  (pad 21 smd rect (at 1.905 -5.461 270) (size 0.381 1.651) (layers F.Cu F.Paste F.Mask) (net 8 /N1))
  (pad 22 smd rect (at 1.27 -5.461 270) (size 0.381 1.651) (layers F.Cu F.Paste F.Mask) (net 7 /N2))
  (pad 23 smd rect (at 0.635 -5.461 270) (size 0.381 1.651) (layers F.Cu F.Paste F.Mask) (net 86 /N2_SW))
  (pad 24 smd rect (at 0 -5.461 270) (size 0.381 1.651) (layers F.Cu F.Paste F.Mask) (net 107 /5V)))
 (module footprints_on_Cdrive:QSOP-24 (layer F.Cu) (at 2.9718 -13.6652 270)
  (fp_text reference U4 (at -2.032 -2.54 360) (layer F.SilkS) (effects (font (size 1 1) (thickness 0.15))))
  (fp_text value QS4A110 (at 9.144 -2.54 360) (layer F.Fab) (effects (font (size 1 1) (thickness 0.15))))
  (pad 1 smd rect (at 0 0 270) (size 0.381 1.651) (layers F.Cu F.Paste F.Mask) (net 108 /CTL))
  (pad 2 smd rect (at 0.635 0 270) (size 0.381 1.651) (layers F.Cu F.Paste F.Mask) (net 87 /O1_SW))
  (pad 3 smd rect (at 1.27 0 270) (size 0.381 1.651) (layers F.Cu F.Paste F.Mask) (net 10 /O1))
  (pad 4 smd rect (at 1.905 0 270) (size 0.381 1.651) (layers F.Cu F.Paste F.Mask) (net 9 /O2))
  (pad 5 smd rect (at 2.54 0 270) (size 0.381 1.651) (layers F.Cu F.Paste F.Mask) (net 92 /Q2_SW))
  (pad 6 smd rect (at 3.175 0 270) (size 0.381 1.651) (layers F.Cu F.Paste F.Mask) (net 89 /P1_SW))
  (pad 7 smd rect (at 3.81 0 270) (size 0.381 1.651) (layers F.Cu F.Paste F.Mask) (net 12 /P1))
  (pad 8 smd rect (at 4.445 0 270) (size 0.381 1.651) (layers F.Cu F.Paste F.Mask) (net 11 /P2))
  (pad 9 smd rect (at 5.08 0 270) (size 0.381 1.651) (layers F.Cu F.Paste F.Mask) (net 90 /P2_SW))
  (pad 10 smd rect (at 5.715 0 270) (size 0.381 1.651) (layers F.Cu F.Paste F.Mask) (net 91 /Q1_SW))
  (pad 11 smd rect (at 6.35 0 270) (size 0.381 1.651) (layers F.Cu F.Paste F.Mask) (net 14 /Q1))
  (pad 12 smd rect (at 6.985 0 270) (size 0.381 1.651) (layers F.Cu F.Paste F.Mask) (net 29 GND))
  (pad 13 smd rect (at 6.985 -5.461 270) (size 0.381 1.651) (layers F.Cu F.Paste F.Mask) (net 108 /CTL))
  (pad 14 smd rect (at 6.35 -5.461 270) (size 0.381 1.651) (layers F.Cu F.Paste F.Mask) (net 13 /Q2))
  (pad 15 smd rect (at 5.715 -5.461 270) (size 0.381 1.651) (layers F.Cu F.Paste F.Mask))
  (pad 16 smd rect (at 5.08 -5.461 270) (size 0.381 1.651) (layers F.Cu F.Paste F.Mask) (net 93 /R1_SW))
  (pad 17 smd rect (at 4.445 -5.461 270) (size 0.381 1.651) (layers F.Cu F.Paste F.Mask) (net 16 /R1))
  (pad 18 smd rect (at 3.81 -5.461 270) (size 0.381 1.651) (layers F.Cu F.Paste F.Mask) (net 15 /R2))
  (pad 19 smd rect (at 3.175 -5.461 270) (size 0.381 1.651) (layers F.Cu F.Paste F.Mask) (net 94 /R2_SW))
  (pad 20 smd rect (at 2.54 -5.461 270) (size 0.381 1.651) (layers F.Cu F.Paste F.Mask) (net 95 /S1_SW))
  (pad 21 smd rect (at 1.905 -5.461 270) (size 0.381 1.651) (layers F.Cu F.Paste F.Mask) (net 18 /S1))
  (pad 22 smd rect (at 1.27 -5.461 270) (size 0.381 1.651) (layers F.Cu F.Paste F.Mask) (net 17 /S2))
  (pad 23 smd rect (at 0.635 -5.461 270) (size 0.381 1.651) (layers F.Cu F.Paste F.Mask) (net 96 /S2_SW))
  (pad 24 smd rect (at 0 -5.461 270) (size 0.381 1.651) (layers F.Cu F.Paste F.Mask) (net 107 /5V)))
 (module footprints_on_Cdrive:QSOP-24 (layer F.Cu) (at 3.3528 -2.2352 270)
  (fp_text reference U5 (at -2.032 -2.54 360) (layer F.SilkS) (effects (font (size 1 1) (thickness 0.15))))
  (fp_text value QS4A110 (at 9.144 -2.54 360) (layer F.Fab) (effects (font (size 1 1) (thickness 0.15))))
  (pad 1 smd rect (at 0 0 270) (size 0.381 1.651) (layers F.Cu F.Paste F.Mask) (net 108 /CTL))
  (pad 2 smd rect (at 0.635 0 270) (size 0.381 1.651) (layers F.Cu F.Paste F.Mask) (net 97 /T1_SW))
  (pad 3 smd rect (at 1.27 0 270) (size 0.381 1.651) (layers F.Cu F.Paste F.Mask) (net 20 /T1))
  (pad 4 smd rect (at 1.905 0 270) (size 0.381 1.651) (layers F.Cu F.Paste F.Mask) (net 19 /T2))
  (pad 5 smd rect (at 2.54 0 270) (size 0.381 1.651) (layers F.Cu F.Paste F.Mask) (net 98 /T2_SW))
  (pad 6 smd rect (at 3.175 0 270) (size 0.381 1.651) (layers F.Cu F.Paste F.Mask) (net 99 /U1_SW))
  (pad 7 smd rect (at 3.81 0 270) (size 0.381 1.651) (layers F.Cu F.Paste F.Mask) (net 22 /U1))
  (pad 8 smd rect (at 4.445 0 270) (size 0.381 1.651) (layers F.Cu F.Paste F.Mask) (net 21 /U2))
  (pad 9 smd rect (at 5.08 0 270) (size 0.381 1.651) (layers F.Cu F.Paste F.Mask) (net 100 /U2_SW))
  (pad 10 smd rect (at 5.715 0 270) (size 0.381 1.651) (layers F.Cu F.Paste F.Mask) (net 101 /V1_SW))
  (pad 11 smd rect (at 6.35 0 270) (size 0.381 1.651) (layers F.Cu F.Paste F.Mask) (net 24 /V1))
  (pad 12 smd rect (at 6.985 0 270) (size 0.381 1.651) (layers F.Cu F.Paste F.Mask) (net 29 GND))
  (pad 13 smd rect (at 6.985 -5.461 270) (size 0.381 1.651) (layers F.Cu F.Paste F.Mask) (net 108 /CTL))
  (pad 14 smd rect (at 6.35 -5.461 270) (size 0.381 1.651) (layers F.Cu F.Paste F.Mask) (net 23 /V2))
  (pad 15 smd rect (at 5.715 -5.461 270) (size 0.381 1.651) (layers F.Cu F.Paste F.Mask))
  (pad 16 smd rect (at 5.08 -5.461 270) (size 0.381 1.651) (layers F.Cu F.Paste F.Mask) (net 103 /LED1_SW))
  (pad 17 smd rect (at 4.445 -5.461 270) (size 0.381 1.651) (layers F.Cu F.Paste F.Mask) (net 28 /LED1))
  (pad 18 smd rect (at 3.81 -5.461 270) (size 0.381 1.651) (layers F.Cu F.Paste F.Mask) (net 25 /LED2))
  (pad 19 smd rect (at 3.175 -5.461 270) (size 0.381 1.651) (layers F.Cu F.Paste F.Mask) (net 104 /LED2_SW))
  (pad 20 smd rect (at 2.54 -5.461 270) (size 0.381 1.651) (layers F.Cu F.Paste F.Mask) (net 105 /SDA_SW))
  (pad 21 smd rect (at 1.905 -5.461 270) (size 0.381 1.651) (layers F.Cu F.Paste F.Mask) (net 27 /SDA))
  (pad 22 smd rect (at 1.27 -5.461 270) (size 0.381 1.651) (layers F.Cu F.Paste F.Mask) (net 30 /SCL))
  (pad 23 smd rect (at 0.635 -5.461 270) (size 0.381 1.651) (layers F.Cu F.Paste F.Mask) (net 106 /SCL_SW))
  (pad 24 smd rect (at 0 -5.461 270) (size 0.381 1.651) (layers F.Cu F.Paste F.Mask) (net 107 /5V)))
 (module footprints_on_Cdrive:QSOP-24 (layer F.Cu) (at -12.6746 -11.8618 270)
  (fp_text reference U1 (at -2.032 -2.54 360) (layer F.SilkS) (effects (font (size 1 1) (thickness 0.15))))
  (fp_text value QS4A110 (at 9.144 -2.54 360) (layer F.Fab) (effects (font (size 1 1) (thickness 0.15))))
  (pad 1 smd rect (at 0 0 270) (size 0.381 1.651) (layers F.Cu F.Paste F.Mask) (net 108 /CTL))
  (pad 2 smd rect (at 0.635 0 270) (size 0.381 1.651) (layers F.Cu F.Paste F.Mask) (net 57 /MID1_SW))
  (pad 3 smd rect (at 1.27 0 270) (size 0.381 1.651) (layers F.Cu F.Paste F.Mask) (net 32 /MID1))
  (pad 4 smd rect (at 1.905 0 270) (size 0.381 1.651) (layers F.Cu F.Paste F.Mask) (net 2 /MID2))
  (pad 5 smd rect (at 2.54 0 270) (size 0.381 1.651) (layers F.Cu F.Paste F.Mask) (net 62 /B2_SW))
  (pad 6 smd rect (at 3.175 0 270) (size 0.381 1.651) (layers F.Cu F.Paste F.Mask) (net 59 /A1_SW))
  (pad 7 smd rect (at 3.81 0 270) (size 0.381 1.651) (layers F.Cu F.Paste F.Mask) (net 34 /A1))
  (pad 8 smd rect (at 4.445 0 270) (size 0.381 1.651) (layers F.Cu F.Paste F.Mask) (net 33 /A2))
  (pad 9 smd rect (at 5.08 0 270) (size 0.381 1.651) (layers F.Cu F.Paste F.Mask) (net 60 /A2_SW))
  (pad 10 smd rect (at 5.715 0 270) (size 0.381 1.651) (layers F.Cu F.Paste F.Mask) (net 61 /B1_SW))
  (pad 11 smd rect (at 6.35 0 270) (size 0.381 1.651) (layers F.Cu F.Paste F.Mask) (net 36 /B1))
  (pad 12 smd rect (at 6.985 0 270) (size 0.381 1.651) (layers F.Cu F.Paste F.Mask) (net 29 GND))
  (pad 13 smd rect (at 6.985 -5.461 270) (size 0.381 1.651) (layers F.Cu F.Paste F.Mask) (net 108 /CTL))
  (pad 14 smd rect (at 6.35 -5.461 270) (size 0.381 1.651) (layers F.Cu F.Paste F.Mask) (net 35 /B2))
  (pad 15 smd rect (at 5.715 -5.461 270) (size 0.381 1.651) (layers F.Cu F.Paste F.Mask))
  (pad 16 smd rect (at 5.08 -5.461 270) (size 0.381 1.651) (layers F.Cu F.Paste F.Mask) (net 63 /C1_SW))
  (pad 17 smd rect (at 4.445 -5.461 270) (size 0.381 1.651) (layers F.Cu F.Paste F.Mask) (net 38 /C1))
  (pad 18 smd rect (at 3.81 -5.461 270) (size 0.381 1.651) (layers F.Cu F.Paste F.Mask) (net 37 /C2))
  (pad 19 smd rect (at 3.175 -5.461 270) (size 0.381 1.651) (layers F.Cu F.Paste F.Mask) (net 64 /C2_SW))
  (pad 20 smd rect (at 2.54 -5.461 270) (size 0.381 1.651) (layers F.Cu F.Paste F.Mask) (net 65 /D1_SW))
  (pad 21 smd rect (at 1.905 -5.461 270) (size 0.381 1.651) (layers F.Cu F.Paste F.Mask) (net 40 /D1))
  (pad 22 smd rect (at 1.27 -5.461 270) (size 0.381 1.651) (layers F.Cu F.Paste F.Mask) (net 39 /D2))
  (pad 23 smd rect (at 0.635 -5.461 270) (size 0.381 1.651) (layers F.Cu F.Paste F.Mask) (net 66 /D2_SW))
  (pad 24 smd rect (at 0 -5.461 270) (size 0.381 1.651) (layers F.Cu F.Paste F.Mask) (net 107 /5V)))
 (gr_line (start 50 -30) (end -50 -30) (angle 90) (layer Edge.Cuts) (width 0.15))
 (gr_line (start 50 -19) (end 50 -30) (angle 90) (layer Edge.Cuts) (width 0.15))
 (gr_line (start -50 -19) (end -50 -30) (angle 90) (layer Edge.Cuts) (width 0.15))
 (gr_line (start 30 -19) (end 50 -19) (angle 90) (layer Edge.Cuts) (width 0.15))
 (gr_line (start -50 -19) (end -30 -19) (angle 90) (layer Edge.Cuts) (width 0.15))
 (gr_line (start -30 -19) (end -30 20) (angle 90) (layer Edge.Cuts) (width 0.15))
 (gr_line (start 30 20) (end 30 -19) (angle 90) (layer Edge.Cuts) (width 0.15))
 (gr_line (start -30 20) (end 30 20) (angle 90) (layer Edge.Cuts) (width 0.15))
 (segment (start -25.865 -12.8) (end -24.622 -11.557) (width 0.1524) (layer B.Cu) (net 32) (status 400000))
 (segment (start -24.622 -11.557) (end -14.0716 -11.557) (width 0.1524) (layer B.Cu) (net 32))
 (segment (start -25.865 -10.26) (end -24.622 -9.017) (width 0.1524) (layer B.Cu) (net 34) (status 400000))
 (segment (start -24.622 -9.017) (end -14.2494 -9.017) (width 0.1524) (layer B.Cu) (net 34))
 (segment (start -23.325 -10.26) (end -14.6034 -10.26) (width 0.1524) (layer B.Cu) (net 33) (status 400000))
 (segment (start -14.6034 -10.26) (end -14.5796 -10.2362) (width 0.1524) (layer B.Cu) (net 33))
 (segment (start -25.865 -7.72) (end -24.622 -6.477) (width 0.1524) (layer B.Cu) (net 36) (status 400000))
 (segment (start -24.622 -6.477) (end -14.5034 -6.477) (width 0.1524) (layer B.Cu) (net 36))
 (segment (start -23.325 -7.72) (end -14.5558 -7.72) (width 0.1524) (layer B.Cu) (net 35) (status 400000))
 (segment (start -14.5558 -7.72) (end -14.5288 -7.747) (width 0.1524) (layer B.Cu) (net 35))
 (segment (start -25.865 -5.18) (end -24.5966 -3.9116) (width 0.1524) (layer B.Cu) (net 38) (status 400000))
 (segment (start -24.5966 -3.9116) (end -14.8082 -3.9116) (width 0.1524) (layer B.Cu) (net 38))
 (segment (start -23.325 -5.18) (end -14.886 -5.18) (width 0.1524) (layer B.Cu) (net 37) (status 400000))
 (segment (start -14.886 -5.18) (end -14.8844 -5.1816) (width 0.1524) (layer B.Cu) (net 37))
 (segment (start -25.865 -2.64) (end -24.622 -1.397) (width 0.1524) (layer B.Cu) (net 40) (status 400000))
 (segment (start -24.622 -1.397) (end -14.4272 -1.397) (width 0.1524) (layer B.Cu) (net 40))
 (segment (start -23.325 -2.64) (end -14.8574 -2.64) (width 0.1524) (layer B.Cu) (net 39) (status 400000))
 (segment (start -14.8574 -2.64) (end -14.8336 -2.6162) (width 0.1524) (layer B.Cu) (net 39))
 (segment (start -25.865 -0.1) (end -24.622 1.143) (width 0.1524) (layer B.Cu) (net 42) (status 400000))
 (segment (start -14.8082 1.143) (end -14.7828 1.1176) (width 0.1524) (layer B.Cu) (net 42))
 (segment (start -24.622 1.143) (end -14.8082 1.143) (width 0.1524) (layer B.Cu) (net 42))
 (segment (start -23.325 -0.1) (end -23.1742 0.0508) (width 0.1524) (layer B.Cu) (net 41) (status C00000))
 (segment (start -23.1742 0.0508) (end -14.9606 0.0508) (width 0.1524) (layer B.Cu) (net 41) (status 400000)))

